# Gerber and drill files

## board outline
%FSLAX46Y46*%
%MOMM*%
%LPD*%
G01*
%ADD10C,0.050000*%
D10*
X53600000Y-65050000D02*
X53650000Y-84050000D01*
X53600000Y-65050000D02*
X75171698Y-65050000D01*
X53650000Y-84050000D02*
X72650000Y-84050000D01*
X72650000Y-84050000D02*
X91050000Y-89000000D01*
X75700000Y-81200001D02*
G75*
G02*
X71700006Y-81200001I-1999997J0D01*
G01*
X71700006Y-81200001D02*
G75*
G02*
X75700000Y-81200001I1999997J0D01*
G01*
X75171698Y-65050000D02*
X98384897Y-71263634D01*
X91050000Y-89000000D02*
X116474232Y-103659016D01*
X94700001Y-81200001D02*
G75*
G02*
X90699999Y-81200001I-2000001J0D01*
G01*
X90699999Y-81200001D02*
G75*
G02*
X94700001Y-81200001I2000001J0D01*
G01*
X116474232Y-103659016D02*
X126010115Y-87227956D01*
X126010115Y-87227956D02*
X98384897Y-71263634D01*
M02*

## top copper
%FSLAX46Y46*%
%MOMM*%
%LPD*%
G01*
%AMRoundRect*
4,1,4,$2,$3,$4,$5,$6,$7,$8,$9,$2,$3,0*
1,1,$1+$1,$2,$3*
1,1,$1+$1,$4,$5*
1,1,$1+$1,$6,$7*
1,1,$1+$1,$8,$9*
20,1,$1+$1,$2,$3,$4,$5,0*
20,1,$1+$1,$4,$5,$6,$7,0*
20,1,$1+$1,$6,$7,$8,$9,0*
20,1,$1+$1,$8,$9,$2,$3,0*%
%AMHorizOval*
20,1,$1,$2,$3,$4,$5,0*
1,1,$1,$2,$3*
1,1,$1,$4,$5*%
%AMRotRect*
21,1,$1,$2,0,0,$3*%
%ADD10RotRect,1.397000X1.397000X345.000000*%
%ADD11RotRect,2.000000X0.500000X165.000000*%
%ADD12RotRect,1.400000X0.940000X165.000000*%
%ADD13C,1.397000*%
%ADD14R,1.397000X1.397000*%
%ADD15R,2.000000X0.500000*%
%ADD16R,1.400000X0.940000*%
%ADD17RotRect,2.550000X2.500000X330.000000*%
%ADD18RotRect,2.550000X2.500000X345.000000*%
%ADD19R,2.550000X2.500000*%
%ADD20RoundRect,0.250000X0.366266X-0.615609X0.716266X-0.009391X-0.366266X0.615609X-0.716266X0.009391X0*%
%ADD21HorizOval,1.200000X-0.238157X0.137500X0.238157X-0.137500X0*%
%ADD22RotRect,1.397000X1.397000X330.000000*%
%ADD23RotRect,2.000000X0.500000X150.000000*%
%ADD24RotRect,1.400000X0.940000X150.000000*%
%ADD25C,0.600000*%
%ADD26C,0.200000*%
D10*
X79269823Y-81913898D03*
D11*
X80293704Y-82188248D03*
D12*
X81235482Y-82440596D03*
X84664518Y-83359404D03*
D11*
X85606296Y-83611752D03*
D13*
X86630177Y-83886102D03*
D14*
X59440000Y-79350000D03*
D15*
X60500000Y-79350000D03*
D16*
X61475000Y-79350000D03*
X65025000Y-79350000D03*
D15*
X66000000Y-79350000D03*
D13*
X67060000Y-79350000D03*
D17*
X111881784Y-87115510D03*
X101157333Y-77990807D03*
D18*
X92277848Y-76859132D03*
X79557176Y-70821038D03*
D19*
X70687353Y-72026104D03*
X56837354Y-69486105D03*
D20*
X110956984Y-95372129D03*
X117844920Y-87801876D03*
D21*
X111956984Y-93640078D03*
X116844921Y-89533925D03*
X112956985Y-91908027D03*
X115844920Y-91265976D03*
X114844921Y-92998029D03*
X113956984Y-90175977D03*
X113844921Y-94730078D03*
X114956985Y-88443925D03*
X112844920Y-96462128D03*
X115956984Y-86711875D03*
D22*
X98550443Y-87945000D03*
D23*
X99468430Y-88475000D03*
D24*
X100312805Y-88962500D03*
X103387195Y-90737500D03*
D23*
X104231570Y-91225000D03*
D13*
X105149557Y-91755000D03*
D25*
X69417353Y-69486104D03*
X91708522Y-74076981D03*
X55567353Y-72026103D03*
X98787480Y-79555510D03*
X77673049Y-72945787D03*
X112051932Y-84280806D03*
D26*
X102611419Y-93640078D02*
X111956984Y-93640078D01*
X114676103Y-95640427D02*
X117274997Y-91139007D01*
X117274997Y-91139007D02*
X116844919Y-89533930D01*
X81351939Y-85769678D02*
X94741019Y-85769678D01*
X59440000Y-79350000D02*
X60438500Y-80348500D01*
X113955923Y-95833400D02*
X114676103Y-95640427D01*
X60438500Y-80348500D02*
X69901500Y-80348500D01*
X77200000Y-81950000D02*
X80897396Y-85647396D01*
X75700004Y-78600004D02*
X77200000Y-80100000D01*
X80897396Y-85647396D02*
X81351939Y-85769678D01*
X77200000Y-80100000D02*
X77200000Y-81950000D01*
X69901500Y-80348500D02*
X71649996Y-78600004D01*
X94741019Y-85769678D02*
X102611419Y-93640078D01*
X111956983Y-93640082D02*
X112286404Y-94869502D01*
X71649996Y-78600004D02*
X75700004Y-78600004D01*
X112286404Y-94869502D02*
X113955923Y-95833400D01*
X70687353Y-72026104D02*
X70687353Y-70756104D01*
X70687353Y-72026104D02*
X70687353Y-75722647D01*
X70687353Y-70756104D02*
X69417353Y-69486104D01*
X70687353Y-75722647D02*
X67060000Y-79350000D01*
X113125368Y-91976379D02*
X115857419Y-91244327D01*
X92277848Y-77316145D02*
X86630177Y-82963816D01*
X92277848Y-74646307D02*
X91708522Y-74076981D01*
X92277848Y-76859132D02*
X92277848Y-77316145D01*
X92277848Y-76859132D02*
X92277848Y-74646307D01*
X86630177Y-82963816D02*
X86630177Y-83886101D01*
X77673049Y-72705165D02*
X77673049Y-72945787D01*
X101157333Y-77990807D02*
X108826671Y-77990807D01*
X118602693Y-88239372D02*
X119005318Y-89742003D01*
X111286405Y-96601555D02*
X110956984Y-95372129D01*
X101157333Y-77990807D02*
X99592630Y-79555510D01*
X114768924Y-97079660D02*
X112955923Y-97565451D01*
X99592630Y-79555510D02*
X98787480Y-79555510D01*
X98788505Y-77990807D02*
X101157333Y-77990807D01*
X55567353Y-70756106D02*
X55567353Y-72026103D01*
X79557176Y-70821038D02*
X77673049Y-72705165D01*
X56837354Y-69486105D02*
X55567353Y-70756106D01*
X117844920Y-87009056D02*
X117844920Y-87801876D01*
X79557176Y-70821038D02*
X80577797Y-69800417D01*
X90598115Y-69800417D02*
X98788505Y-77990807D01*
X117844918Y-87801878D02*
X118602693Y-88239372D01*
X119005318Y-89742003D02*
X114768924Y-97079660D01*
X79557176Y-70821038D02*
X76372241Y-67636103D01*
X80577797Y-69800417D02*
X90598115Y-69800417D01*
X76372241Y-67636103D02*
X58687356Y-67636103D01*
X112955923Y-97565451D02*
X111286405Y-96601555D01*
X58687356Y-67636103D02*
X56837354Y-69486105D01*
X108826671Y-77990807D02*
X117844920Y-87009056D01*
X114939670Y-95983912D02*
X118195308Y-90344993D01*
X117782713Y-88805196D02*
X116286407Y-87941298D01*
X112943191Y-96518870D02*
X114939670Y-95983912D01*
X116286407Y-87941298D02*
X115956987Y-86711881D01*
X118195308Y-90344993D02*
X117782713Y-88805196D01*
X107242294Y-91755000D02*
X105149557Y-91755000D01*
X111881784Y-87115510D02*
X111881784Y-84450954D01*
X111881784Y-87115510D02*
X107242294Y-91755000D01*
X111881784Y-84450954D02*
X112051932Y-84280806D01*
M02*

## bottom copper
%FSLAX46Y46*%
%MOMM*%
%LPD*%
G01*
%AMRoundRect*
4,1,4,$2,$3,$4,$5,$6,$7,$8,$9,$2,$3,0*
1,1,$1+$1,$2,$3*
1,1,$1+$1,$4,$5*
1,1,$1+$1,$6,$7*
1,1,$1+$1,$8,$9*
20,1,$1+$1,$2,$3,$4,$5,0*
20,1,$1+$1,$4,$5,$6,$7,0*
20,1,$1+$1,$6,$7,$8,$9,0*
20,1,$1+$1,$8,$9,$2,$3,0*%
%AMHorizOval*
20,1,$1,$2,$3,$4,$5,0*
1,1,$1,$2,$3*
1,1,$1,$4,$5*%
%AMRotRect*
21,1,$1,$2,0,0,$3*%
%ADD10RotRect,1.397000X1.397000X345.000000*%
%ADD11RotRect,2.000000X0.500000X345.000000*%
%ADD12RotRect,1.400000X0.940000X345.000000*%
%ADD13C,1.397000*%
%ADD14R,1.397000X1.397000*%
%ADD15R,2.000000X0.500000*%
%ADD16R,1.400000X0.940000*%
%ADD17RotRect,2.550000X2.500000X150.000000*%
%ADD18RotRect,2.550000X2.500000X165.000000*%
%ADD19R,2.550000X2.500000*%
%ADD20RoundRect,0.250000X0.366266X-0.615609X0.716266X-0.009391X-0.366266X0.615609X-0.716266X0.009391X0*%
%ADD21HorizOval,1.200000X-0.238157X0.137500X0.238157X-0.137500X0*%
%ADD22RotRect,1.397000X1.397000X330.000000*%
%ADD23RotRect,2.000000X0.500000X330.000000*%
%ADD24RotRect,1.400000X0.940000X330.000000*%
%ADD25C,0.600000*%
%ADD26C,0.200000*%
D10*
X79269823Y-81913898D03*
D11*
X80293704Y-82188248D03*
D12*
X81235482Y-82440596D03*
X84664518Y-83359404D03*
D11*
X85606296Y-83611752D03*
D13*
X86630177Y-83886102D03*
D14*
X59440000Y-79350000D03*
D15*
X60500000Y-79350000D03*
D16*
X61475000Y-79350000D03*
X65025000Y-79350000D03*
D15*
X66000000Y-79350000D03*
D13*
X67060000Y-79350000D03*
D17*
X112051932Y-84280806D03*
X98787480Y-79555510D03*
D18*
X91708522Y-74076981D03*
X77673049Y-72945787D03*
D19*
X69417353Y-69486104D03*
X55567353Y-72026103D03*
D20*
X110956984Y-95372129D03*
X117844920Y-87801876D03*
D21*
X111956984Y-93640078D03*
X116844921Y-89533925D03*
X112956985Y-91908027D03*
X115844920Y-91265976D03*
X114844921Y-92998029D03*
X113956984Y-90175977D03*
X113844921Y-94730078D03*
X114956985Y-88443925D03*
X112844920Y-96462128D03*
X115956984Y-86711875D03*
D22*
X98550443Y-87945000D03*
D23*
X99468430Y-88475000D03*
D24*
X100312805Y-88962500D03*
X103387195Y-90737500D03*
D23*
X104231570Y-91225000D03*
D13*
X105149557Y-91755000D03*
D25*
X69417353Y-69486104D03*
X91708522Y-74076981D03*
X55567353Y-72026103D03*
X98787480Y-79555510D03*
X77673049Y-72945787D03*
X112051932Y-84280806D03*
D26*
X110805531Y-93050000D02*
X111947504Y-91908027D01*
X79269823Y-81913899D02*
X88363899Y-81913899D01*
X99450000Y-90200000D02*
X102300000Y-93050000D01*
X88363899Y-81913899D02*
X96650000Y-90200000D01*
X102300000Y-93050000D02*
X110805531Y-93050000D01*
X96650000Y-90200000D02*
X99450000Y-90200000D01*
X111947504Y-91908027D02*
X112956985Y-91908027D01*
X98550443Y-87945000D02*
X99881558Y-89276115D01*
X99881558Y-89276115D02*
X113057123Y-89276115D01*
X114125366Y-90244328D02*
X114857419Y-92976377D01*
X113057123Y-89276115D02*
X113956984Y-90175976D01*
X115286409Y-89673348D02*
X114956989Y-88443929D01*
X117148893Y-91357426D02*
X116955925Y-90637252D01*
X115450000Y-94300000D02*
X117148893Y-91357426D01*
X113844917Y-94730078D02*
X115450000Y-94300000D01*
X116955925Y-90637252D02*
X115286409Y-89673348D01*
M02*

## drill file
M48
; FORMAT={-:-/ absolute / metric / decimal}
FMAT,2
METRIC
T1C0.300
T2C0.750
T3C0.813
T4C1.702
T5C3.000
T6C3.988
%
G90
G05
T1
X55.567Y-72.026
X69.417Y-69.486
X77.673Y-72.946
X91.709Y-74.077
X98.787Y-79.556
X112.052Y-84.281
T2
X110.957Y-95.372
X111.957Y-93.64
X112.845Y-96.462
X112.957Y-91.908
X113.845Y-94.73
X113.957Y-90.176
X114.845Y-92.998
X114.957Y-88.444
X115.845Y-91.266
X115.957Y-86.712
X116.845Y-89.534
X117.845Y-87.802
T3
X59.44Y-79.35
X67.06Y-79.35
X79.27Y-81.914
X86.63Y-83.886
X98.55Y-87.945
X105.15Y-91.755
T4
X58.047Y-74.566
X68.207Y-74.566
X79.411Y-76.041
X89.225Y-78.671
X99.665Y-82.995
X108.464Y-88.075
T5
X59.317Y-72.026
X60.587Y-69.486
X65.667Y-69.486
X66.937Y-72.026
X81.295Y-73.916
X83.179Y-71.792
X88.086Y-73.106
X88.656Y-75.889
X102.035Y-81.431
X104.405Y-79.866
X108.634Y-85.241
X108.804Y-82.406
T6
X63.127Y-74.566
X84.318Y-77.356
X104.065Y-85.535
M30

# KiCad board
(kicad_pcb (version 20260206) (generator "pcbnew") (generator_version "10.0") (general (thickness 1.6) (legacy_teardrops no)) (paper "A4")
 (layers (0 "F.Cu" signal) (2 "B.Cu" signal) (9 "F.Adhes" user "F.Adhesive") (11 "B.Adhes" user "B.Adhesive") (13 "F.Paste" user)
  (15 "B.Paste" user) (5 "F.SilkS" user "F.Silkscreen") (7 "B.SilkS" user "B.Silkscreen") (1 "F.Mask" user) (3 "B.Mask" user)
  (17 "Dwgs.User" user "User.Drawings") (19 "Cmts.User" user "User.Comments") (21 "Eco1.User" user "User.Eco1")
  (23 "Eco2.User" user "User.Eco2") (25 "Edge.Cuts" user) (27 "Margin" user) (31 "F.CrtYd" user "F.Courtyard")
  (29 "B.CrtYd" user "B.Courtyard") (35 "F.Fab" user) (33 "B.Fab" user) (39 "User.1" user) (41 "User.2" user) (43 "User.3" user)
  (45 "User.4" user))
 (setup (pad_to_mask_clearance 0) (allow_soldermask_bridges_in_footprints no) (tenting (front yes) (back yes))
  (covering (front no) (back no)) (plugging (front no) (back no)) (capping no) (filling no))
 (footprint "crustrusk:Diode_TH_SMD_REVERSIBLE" (layer "F.Cu") (at 82.95 82.9 -15)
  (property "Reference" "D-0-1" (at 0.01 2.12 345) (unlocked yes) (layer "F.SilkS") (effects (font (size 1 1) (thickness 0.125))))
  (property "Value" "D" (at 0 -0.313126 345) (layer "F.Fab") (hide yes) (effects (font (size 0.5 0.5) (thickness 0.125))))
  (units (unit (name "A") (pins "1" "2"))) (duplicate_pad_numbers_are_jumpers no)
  (pad "1" thru_hole rect (at -3.81 -0.000001 345) (size 1.397 1.397) (drill 0.8128) (layers "*.Cu" "*.Mask") (remove_unused_layers no)
   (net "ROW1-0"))
  (pad "1" smd rect (at -2.75 0 165) (size 2 0.5) (layers "F.Cu") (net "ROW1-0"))
  (pad "1" smd rect (at -2.75 0 345) (size 2 0.5) (layers "B.Cu") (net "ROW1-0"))
  (pad "1" smd rect (at -1.775 0 165) (size 1.4 0.94) (layers "F.Cu" "F.Mask" "F.Paste") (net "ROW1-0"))
  (pad "1" smd rect (at -1.775 0 345) (size 1.4 0.94) (layers "B.Cu" "B.Mask" "B.Paste") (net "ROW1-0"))
  (pad "2" smd rect (at 1.775 0 165) (size 1.4 0.94) (layers "F.Cu" "F.Mask" "F.Paste") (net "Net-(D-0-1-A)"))
  (pad "2" smd rect (at 1.775 0 345) (size 1.4 0.94) (layers "B.Cu" "B.Mask" "B.Paste") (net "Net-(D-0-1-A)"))
  (pad "2" smd rect (at 2.75 0 165) (size 2 0.5) (layers "F.Cu") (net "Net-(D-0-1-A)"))
  (pad "2" smd rect (at 2.75 0 345) (size 2 0.5) (layers "B.Cu") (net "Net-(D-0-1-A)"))
  (pad "2" thru_hole circle (at 3.81 0.000001 345) (size 1.397 1.397) (drill 0.8128) (layers "*.Cu" "*.Mask") (remove_unused_layers no)
   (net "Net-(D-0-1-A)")))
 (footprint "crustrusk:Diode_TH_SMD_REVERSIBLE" (layer "F.Cu") (at 63.25 79.35)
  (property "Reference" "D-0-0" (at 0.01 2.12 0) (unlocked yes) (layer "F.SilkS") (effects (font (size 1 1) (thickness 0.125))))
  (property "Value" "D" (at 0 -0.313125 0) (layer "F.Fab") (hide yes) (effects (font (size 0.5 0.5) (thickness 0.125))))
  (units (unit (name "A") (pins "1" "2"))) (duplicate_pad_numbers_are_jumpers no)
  (pad "1" thru_hole rect (at -3.81 0) (size 1.397 1.397) (drill 0.8128) (layers "*.Cu" "*.Mask") (remove_unused_layers no) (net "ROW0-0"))
  (pad "1" smd rect (at -2.75 0 180) (size 2 0.5) (layers "F.Cu") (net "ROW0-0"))
  (pad "1" smd rect (at -2.75 0) (size 2 0.5) (layers "B.Cu") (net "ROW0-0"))
  (pad "1" smd rect (at -1.775 0 180) (size 1.4 0.94) (layers "F.Cu" "F.Mask" "F.Paste") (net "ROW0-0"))
  (pad "1" smd rect (at -1.775 0) (size 1.4 0.94) (layers "B.Cu" "B.Mask" "B.Paste") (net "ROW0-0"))
  (pad "2" smd rect (at 1.775 0 180) (size 1.4 0.94) (layers "F.Cu" "F.Mask" "F.Paste") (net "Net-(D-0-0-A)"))
  (pad "2" smd rect (at 1.775 0) (size 1.4 0.94) (layers "B.Cu" "B.Mask" "B.Paste") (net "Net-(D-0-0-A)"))
  (pad "2" smd rect (at 2.75 0 180) (size 2 0.5) (layers "F.Cu") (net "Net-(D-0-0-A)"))
  (pad "2" smd rect (at 2.75 0) (size 2 0.5) (layers "B.Cu") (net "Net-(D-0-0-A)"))
  (pad "2" thru_hole circle (at 3.81 0) (size 1.397 1.397) (drill 0.8128) (layers "*.Cu" "*.Mask") (remove_unused_layers no)
   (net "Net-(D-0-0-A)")))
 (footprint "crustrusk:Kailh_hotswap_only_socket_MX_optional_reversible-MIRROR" (layer "F.Cu") (at 104.064632 85.535215 -30)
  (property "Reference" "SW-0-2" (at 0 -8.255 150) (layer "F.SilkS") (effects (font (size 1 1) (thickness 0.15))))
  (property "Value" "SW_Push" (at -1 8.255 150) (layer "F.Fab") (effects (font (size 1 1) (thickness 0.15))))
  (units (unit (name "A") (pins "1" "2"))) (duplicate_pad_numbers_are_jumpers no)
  (pad "" np_thru_hole circle (at -5.08 0 330) (size 1.7018 1.7018) (drill 1.7018) (layers "*.Cu" "*.Mask"))
  (pad "" np_thru_hole circle (at -3.81 -2.54 150) (size 3 3) (drill 3) (layers "*.Cu" "*.Mask"))
  (pad "" np_thru_hole circle (at -2.54 -5.079997 330) (size 3 3) (drill 3) (layers "*.Cu" "*.Mask"))
  (pad "" np_thru_hole circle (at 0 0 330) (size 3.9878 3.9878) (drill 3.9878) (layers "*.Cu" "*.Mask"))
  (pad "" np_thru_hole circle (at 2.540002 -5.080001 150) (size 3 3) (drill 3) (layers "*.Cu" "*.Mask"))
  (pad "" np_thru_hole circle (at 3.81 -2.540001 330) (size 3 3) (drill 3) (layers "*.Cu" "*.Mask"))
  (pad "" np_thru_hole circle (at 5.08 0 330) (size 1.7018 1.7018) (drill 1.7018) (layers "*.Cu" "*.Mask"))
  (pad "1" smd rect (at 6.29 -5.08 150) (size 2.55 2.5) (layers "B.Cu" "B.Mask" "B.Paste") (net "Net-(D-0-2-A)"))
  (pad "1" smd rect (at 7.56 -2.54 330) (size 2.55 2.5) (layers "F.Cu" "F.Mask" "F.Paste") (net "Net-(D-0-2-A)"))
  (pad "2" smd rect (at -7.56 -2.54 150) (size 2.55 2.5) (layers "B.Cu" "B.Mask" "B.Paste") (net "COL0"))
  (pad "2" smd rect (at -6.289999 -5.079999 330) (size 2.55 2.5) (layers "F.Cu" "F.Mask" "F.Paste") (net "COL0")))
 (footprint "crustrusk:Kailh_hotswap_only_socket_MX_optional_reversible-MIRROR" (layer "F.Cu") (at 84.318048 77.355912 -15)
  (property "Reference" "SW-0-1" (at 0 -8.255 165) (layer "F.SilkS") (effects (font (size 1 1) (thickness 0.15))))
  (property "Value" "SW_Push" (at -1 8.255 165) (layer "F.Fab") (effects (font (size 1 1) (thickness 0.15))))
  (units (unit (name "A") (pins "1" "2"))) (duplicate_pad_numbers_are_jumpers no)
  (pad "" np_thru_hole circle (at -5.08 0 345) (size 1.7018 1.7018) (drill 1.7018) (layers "*.Cu" "*.Mask"))
  (pad "" np_thru_hole circle (at -3.81 -2.54 165) (size 3 3) (drill 3) (layers "*.Cu" "*.Mask"))
  (pad "" np_thru_hole circle (at -2.54 -5.079998 345) (size 3 3) (drill 3) (layers "*.Cu" "*.Mask"))
  (pad "" np_thru_hole circle (at 0 0 345) (size 3.9878 3.9878) (drill 3.9878) (layers "*.Cu" "*.Mask"))
  (pad "" np_thru_hole circle (at 2.540003 -5.080001 165) (size 3 3) (drill 3) (layers "*.Cu" "*.Mask"))
  (pad "" np_thru_hole circle (at 3.81 -2.54 345) (size 3 3) (drill 3) (layers "*.Cu" "*.Mask"))
  (pad "" np_thru_hole circle (at 5.08 0 345) (size 1.7018 1.7018) (drill 1.7018) (layers "*.Cu" "*.Mask"))
  (pad "1" smd rect (at 6.29 -5.08 165) (size 2.55 2.5) (layers "B.Cu" "B.Mask" "B.Paste") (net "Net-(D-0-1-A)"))
  (pad "1" smd rect (at 7.56 -2.54 345) (size 2.55 2.5) (layers "F.Cu" "F.Mask" "F.Paste") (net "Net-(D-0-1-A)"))
  (pad "2" smd rect (at -7.56 -2.540001 165) (size 2.55 2.5) (layers "B.Cu" "B.Mask" "B.Paste") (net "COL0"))
  (pad "2" smd rect (at -6.289999 -5.079999 345) (size 2.55 2.5) (layers "F.Cu" "F.Mask" "F.Paste") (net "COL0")))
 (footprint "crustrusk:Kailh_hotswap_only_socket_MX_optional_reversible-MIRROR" (layer "F.Cu") (at 63.127353 74.566104)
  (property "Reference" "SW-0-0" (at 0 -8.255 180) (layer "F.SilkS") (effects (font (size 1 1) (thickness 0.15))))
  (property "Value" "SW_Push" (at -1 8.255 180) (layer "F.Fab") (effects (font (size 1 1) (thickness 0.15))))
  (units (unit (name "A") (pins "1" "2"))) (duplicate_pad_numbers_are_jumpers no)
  (pad "" np_thru_hole circle (at -5.08 0) (size 1.7018 1.7018) (drill 1.7018) (layers "*.Cu" "*.Mask"))
  (pad "" np_thru_hole circle (at -3.81 -2.54 180) (size 3 3) (drill 3) (layers "*.Cu" "*.Mask"))
  (pad "" np_thru_hole circle (at -2.54 -5.079998) (size 3 3) (drill 3) (layers "*.Cu" "*.Mask"))
  (pad "" np_thru_hole circle (at 0 0) (size 3.9878 3.9878) (drill 3.9878) (layers "*.Cu" "*.Mask"))
  (pad "" np_thru_hole circle (at 2.540002 -5.080001 180) (size 3 3) (drill 3) (layers "*.Cu" "*.Mask"))
  (pad "" np_thru_hole circle (at 3.81 -2.54) (size 3 3) (drill 3) (layers "*.Cu" "*.Mask"))
  (pad "" np_thru_hole circle (at 5.08 0) (size 1.7018 1.7018) (drill 1.7018) (layers "*.Cu" "*.Mask"))
  (pad "1" smd rect (at 6.29 -5.08 180) (size 2.55 2.5) (layers "B.Cu" "B.Mask" "B.Paste") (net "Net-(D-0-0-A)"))
  (pad "1" smd rect (at 7.56 -2.54) (size 2.55 2.5) (layers "F.Cu" "F.Mask" "F.Paste") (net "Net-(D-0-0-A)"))
  (pad "2" smd rect (at -7.56 -2.540001 180) (size 2.55 2.5) (layers "B.Cu" "B.Mask" "B.Paste") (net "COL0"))
  (pad "2" smd rect (at -6.289999 -5.079999) (size 2.55 2.5) (layers "F.Cu" "F.Mask" "F.Paste") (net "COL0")))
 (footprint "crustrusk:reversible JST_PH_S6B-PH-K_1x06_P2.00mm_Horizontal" (layer "F.Cu") (at 110.956984 95.372129 60)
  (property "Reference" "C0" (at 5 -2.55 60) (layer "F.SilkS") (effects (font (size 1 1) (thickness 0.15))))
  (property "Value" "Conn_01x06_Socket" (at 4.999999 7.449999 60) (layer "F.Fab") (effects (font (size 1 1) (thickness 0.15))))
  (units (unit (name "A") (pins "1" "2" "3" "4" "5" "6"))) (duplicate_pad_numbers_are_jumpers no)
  (pad "1" thru_hole roundrect (at 0 0 60) (size 1.2 1.75) (drill 0.75) (layers "*.Cu" "*.Mask") (remove_unused_layers no)
   (roundrect_rratio 0.208333) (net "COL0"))
  (pad "1" thru_hole roundrect (at 9.999999 2.180001 60) (size 1.2 1.75) (drill 0.75) (layers "*.Cu" "*.Mask") (remove_unused_layers no)
   (roundrect_rratio 0.208333) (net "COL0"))
  (pad "2" thru_hole oval (at 2 0 60) (size 1.2 1.75) (drill 0.75) (layers "*.Cu" "*.Mask") (remove_unused_layers no) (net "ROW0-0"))
  (pad "2" thru_hole oval (at 8.000001 2.180001 60) (size 1.2 1.75) (drill 0.75) (layers "*.Cu" "*.Mask") (remove_unused_layers no)
   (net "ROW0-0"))
  (pad "3" thru_hole oval (at 4.000001 0.000001 60) (size 1.2 1.75) (drill 0.75) (layers "*.Cu" "*.Mask") (remove_unused_layers no)
   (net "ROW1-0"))
  (pad "3" thru_hole oval (at 6.000001 2.18 60) (size 1.2 1.75) (drill 0.75) (layers "*.Cu" "*.Mask") (remove_unused_layers no)
   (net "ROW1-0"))
  (pad "4" thru_hole oval (at 3.999999 2.180002 60) (size 1.2 1.75) (drill 0.75) (layers "*.Cu" "*.Mask") (remove_unused_layers no)
   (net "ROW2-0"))
  (pad "4" thru_hole oval (at 6 0 60) (size 1.2 1.75) (drill 0.75) (layers "*.Cu" "*.Mask") (remove_unused_layers no) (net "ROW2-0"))
  (pad "5" thru_hole oval (at 2.000001 2.180001 60) (size 1.2 1.75) (drill 0.75) (layers "*.Cu" "*.Mask") (remove_unused_layers no)
   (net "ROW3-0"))
  (pad "5" thru_hole oval (at 8.000001 0 60) (size 1.2 1.75) (drill 0.75) (layers "*.Cu" "*.Mask") (remove_unused_layers no) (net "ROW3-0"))
  (pad "6" thru_hole oval (at 0.000001 2.18 60) (size 1.2 1.75) (drill 0.75) (layers "*.Cu" "*.Mask") (remove_unused_layers no)
   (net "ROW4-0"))
  (pad "6" thru_hole oval (at 10 0 60) (size 1.2 1.75) (drill 0.75) (layers "*.Cu" "*.Mask") (remove_unused_layers no) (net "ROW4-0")))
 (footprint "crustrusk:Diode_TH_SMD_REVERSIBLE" (layer "F.Cu") (at 101.85 89.85 -30)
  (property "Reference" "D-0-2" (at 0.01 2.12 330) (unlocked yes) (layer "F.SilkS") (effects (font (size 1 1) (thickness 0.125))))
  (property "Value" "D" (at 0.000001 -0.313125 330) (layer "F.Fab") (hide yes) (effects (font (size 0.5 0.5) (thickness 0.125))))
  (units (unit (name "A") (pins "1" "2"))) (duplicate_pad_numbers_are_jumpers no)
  (pad "1" thru_hole rect (at -3.81 0 330) (size 1.397 1.397) (drill 0.8128) (layers "*.Cu" "*.Mask") (remove_unused_layers no)
   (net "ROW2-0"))
  (pad "1" smd rect (at -2.75 0 150) (size 2 0.5) (layers "F.Cu") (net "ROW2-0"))
  (pad "1" smd rect (at -2.75 0 330) (size 2 0.5) (layers "B.Cu") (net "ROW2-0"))
  (pad "1" smd rect (at -1.775 0 150) (size 1.4 0.94) (layers "F.Cu" "F.Mask" "F.Paste") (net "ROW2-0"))
  (pad "1" smd rect (at -1.775 0 330) (size 1.4 0.94) (layers "B.Cu" "B.Mask" "B.Paste") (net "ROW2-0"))
  (pad "2" smd rect (at 1.775 0 150) (size 1.4 0.94) (layers "F.Cu" "F.Mask" "F.Paste") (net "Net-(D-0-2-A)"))
  (pad "2" smd rect (at 1.775 0 330) (size 1.4 0.94) (layers "B.Cu" "B.Mask" "B.Paste") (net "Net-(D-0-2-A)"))
  (pad "2" smd rect (at 2.75 0 150) (size 2 0.5) (layers "F.Cu") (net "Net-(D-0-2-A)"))
  (pad "2" smd rect (at 2.75 0 330) (size 2 0.5) (layers "B.Cu") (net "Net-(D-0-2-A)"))
  (pad "2" thru_hole circle (at 3.81 0 330) (size 1.397 1.397) (drill 0.8128) (layers "*.Cu" "*.Mask") (remove_unused_layers no)
   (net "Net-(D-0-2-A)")))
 (gr_line (start 53.6 65.05) (end 53.65 84.05) (stroke (width 0.05) (type default)) (layer "Edge.Cuts"))
 (gr_line (start 53.6 65.05) (end 75.171698 65.05) (stroke (width 0.05) (type default)) (layer "Edge.Cuts"))
 (gr_line (start 53.65 84.05) (end 72.65 84.05) (stroke (width 0.05) (type default)) (layer "Edge.Cuts"))
 (gr_line (start 72.65 84.05) (end 91.05 89) (stroke (width 0.05) (type default)) (layer "Edge.Cuts"))
 (gr_circle (center 73.700003 81.200001) (end 75.7 81.200001) (stroke (width 0.05) (type default)) (fill no) (layer "Edge.Cuts"))
 (gr_line (start 75.171698 65.05) (end 98.384897 71.263634) (stroke (width 0.05) (type default)) (layer "Edge.Cuts"))
 (gr_line (start 91.05 89) (end 116.474232 103.659016) (stroke (width 0.05) (type default)) (layer "Edge.Cuts"))
 (gr_circle (center 92.7 81.200001) (end 94.700001 81.200001) (stroke (width 0.05) (type default)) (fill no) (layer "Edge.Cuts"))
 (gr_line (start 116.474232 103.659016) (end 126.010115 87.227956) (stroke (width 0.05) (type default)) (layer "Edge.Cuts"))
 (gr_line (start 126.010115 87.227956) (end 98.384897 71.263634) (stroke (width 0.05) (type default)) (layer "Edge.Cuts"))
 (segment (start 102.611419 93.640078) (end 111.956984 93.640078) (width 0.2) (layer "F.Cu") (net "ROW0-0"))
 (segment (start 114.676103 95.640427) (end 117.274997 91.139007) (width 0.2) (layer "F.Cu") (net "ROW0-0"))
 (segment (start 117.274997 91.139007) (end 116.844919 89.53393) (width 0.2) (layer "F.Cu") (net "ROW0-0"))
 (segment (start 81.351939 85.769678) (end 94.741019 85.769678) (width 0.2) (layer "F.Cu") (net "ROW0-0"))
 (segment (start 59.44 79.35) (end 60.4385 80.3485) (width 0.2) (layer "F.Cu") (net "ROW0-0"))
 (segment (start 113.955923 95.8334) (end 114.676103 95.640427) (width 0.2) (layer "F.Cu") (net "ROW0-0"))
 (segment (start 60.4385 80.3485) (end 69.9015 80.3485) (width 0.2) (layer "F.Cu") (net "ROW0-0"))
 (segment (start 77.2 81.95) (end 80.897396 85.647396) (width 0.2) (layer "F.Cu") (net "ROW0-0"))
 (segment (start 75.700004 78.600004) (end 77.2 80.1) (width 0.2) (layer "F.Cu") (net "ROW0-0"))
 (segment (start 80.897396 85.647396) (end 81.351939 85.769678) (width 0.2) (layer "F.Cu") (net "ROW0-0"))
 (segment (start 77.2 80.1) (end 77.2 81.95) (width 0.2) (layer "F.Cu") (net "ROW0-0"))
 (segment (start 69.9015 80.3485) (end 71.649996 78.600004) (width 0.2) (layer "F.Cu") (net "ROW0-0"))
 (segment (start 94.741019 85.769678) (end 102.611419 93.640078) (width 0.2) (layer "F.Cu") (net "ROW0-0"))
 (segment (start 111.956983 93.640082) (end 112.286404 94.869502) (width 0.2) (layer "F.Cu") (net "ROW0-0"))
 (segment (start 71.649996 78.600004) (end 75.700004 78.600004) (width 0.2) (layer "F.Cu") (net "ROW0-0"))
 (segment (start 112.286404 94.869502) (end 113.955923 95.8334) (width 0.2) (layer "F.Cu") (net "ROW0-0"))
 (segment (start 70.687353 72.026104) (end 70.687353 70.756104) (width 0.2) (layer "F.Cu") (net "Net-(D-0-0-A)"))
 (segment (start 70.687353 72.026104) (end 70.687353 75.722647) (width 0.2) (layer "F.Cu") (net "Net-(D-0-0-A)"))
 (segment (start 70.687353 70.756104) (end 69.417353 69.486104) (width 0.2) (layer "F.Cu") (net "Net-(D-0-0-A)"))
 (segment (start 70.687353 75.722647) (end 67.06 79.35) (width 0.2) (layer "F.Cu") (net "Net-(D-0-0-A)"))
 (via (at 69.417353 69.486104) (size 0.6) (drill 0.3) (layers "F.Cu" "B.Cu") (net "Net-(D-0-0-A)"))
 (segment (start 113.125368 91.976379) (end 115.857419 91.244327) (width 0.2) (layer "F.Cu") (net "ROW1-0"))
 (segment (start 110.805531 93.05) (end 111.947504 91.908027) (width 0.2) (layer "B.Cu") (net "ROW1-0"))
 (segment (start 79.269823 81.913899) (end 88.363899 81.913899) (width 0.2) (layer "B.Cu") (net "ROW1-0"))
 (segment (start 99.45 90.2) (end 102.3 93.05) (width 0.2) (layer "B.Cu") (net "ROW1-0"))
 (segment (start 88.363899 81.913899) (end 96.65 90.2) (width 0.2) (layer "B.Cu") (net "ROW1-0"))
 (segment (start 102.3 93.05) (end 110.805531 93.05) (width 0.2) (layer "B.Cu") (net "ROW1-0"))
 (segment (start 96.65 90.2) (end 99.45 90.2) (width 0.2) (layer "B.Cu") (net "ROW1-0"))
 (segment (start 111.947504 91.908027) (end 112.956985 91.908027) (width 0.2) (layer "B.Cu") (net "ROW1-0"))
 (segment (start 92.277848 77.316145) (end 86.630177 82.963816) (width 0.2) (layer "F.Cu") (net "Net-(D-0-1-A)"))
 (segment (start 92.277848 74.646307) (end 91.708522 74.076981) (width 0.2) (layer "F.Cu") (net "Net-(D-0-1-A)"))
 (segment (start 92.277848 76.859132) (end 92.277848 77.316145) (width 0.2) (layer "F.Cu") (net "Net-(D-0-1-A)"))
 (segment (start 92.277848 76.859132) (end 92.277848 74.646307) (width 0.2) (layer "F.Cu") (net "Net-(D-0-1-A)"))
 (segment (start 86.630177 82.963816) (end 86.630177 83.886101) (width 0.2) (layer "F.Cu") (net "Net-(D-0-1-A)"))
 (via (at 91.708522 74.076981) (size 0.6) (drill 0.3) (layers "F.Cu" "B.Cu") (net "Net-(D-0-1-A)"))
 (segment (start 77.673049 72.705165) (end 77.673049 72.945787) (width 0.2) (layer "F.Cu") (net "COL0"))
 (segment (start 101.157333 77.990807) (end 108.826671 77.990807) (width 0.2) (layer "F.Cu") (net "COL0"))
 (segment (start 118.602693 88.239372) (end 119.005318 89.742003) (width 0.2) (layer "F.Cu") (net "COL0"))
 (segment (start 111.286405 96.601555) (end 110.956984 95.372129) (width 0.2) (layer "F.Cu") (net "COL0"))
 (segment (start 101.157333 77.990807) (end 99.59263 79.55551) (width 0.2) (layer "F.Cu") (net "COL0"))
 (segment (start 114.768924 97.07966) (end 112.955923 97.565451) (width 0.2) (layer "F.Cu") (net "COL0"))
 (segment (start 99.59263 79.55551) (end 98.78748 79.55551) (width 0.2) (layer "F.Cu") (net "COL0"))
 (segment (start 98.788505 77.990807) (end 101.157333 77.990807) (width 0.2) (layer "F.Cu") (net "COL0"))
 (segment (start 55.567353 70.756106) (end 55.567353 72.026103) (width 0.2) (layer "F.Cu") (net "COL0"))
 (segment (start 79.557176 70.821038) (end 77.673049 72.705165) (width 0.2) (layer "F.Cu") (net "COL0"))
 (segment (start 56.837354 69.486105) (end 55.567353 70.756106) (width 0.2) (layer "F.Cu") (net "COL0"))
 (segment (start 117.84492 87.009056) (end 117.84492 87.801876) (width 0.2) (layer "F.Cu") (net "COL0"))
 (segment (start 79.557176 70.821038) (end 80.577797 69.800417) (width 0.2) (layer "F.Cu") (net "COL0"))
 (segment (start 90.598115 69.800417) (end 98.788505 77.990807) (width 0.2) (layer "F.Cu") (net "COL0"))
 (segment (start 117.844918 87.801878) (end 118.602693 88.239372) (width 0.2) (layer "F.Cu") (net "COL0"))
 (segment (start 119.005318 89.742003) (end 114.768924 97.07966) (width 0.2) (layer "F.Cu") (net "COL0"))
 (segment (start 79.557176 70.821038) (end 76.372241 67.636103) (width 0.2) (layer "F.Cu") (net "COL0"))
 (segment (start 80.577797 69.800417) (end 90.598115 69.800417) (width 0.2) (layer "F.Cu") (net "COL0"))
 (segment (start 76.372241 67.636103) (end 58.687356 67.636103) (width 0.2) (layer "F.Cu") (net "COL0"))
 (segment (start 112.955923 97.565451) (end 111.286405 96.601555) (width 0.2) (layer "F.Cu") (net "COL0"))
 (segment (start 58.687356 67.636103) (end 56.837354 69.486105) (width 0.2) (layer "F.Cu") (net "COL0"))
 (segment (start 108.826671 77.990807) (end 117.84492 87.009056) (width 0.2) (layer "F.Cu") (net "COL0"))
 (via (at 55.567353 72.026103) (size 0.6) (drill 0.3) (layers "F.Cu" "B.Cu") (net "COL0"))
 (via (at 98.78748 79.55551) (size 0.6) (drill 0.3) (layers "F.Cu" "B.Cu") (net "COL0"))
 (via (at 77.673049 72.945787) (size 0.6) (drill 0.3) (layers "F.Cu" "B.Cu") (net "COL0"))
 (segment (start 98.550443 87.945) (end 99.881558 89.276115) (width 0.2) (layer "B.Cu") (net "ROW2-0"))
 (segment (start 99.881558 89.276115) (end 113.057123 89.276115) (width 0.2) (layer "B.Cu") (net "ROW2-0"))
 (segment (start 114.125366 90.244328) (end 114.857419 92.976377) (width 0.2) (layer "B.Cu") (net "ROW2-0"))
 (segment (start 113.057123 89.276115) (end 113.956984 90.175976) (width 0.2) (layer "B.Cu") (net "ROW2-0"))
 (segment (start 115.286409 89.673348) (end 114.956989 88.443929) (width 0.2) (layer "B.Cu") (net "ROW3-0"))
 (segment (start 117.148893 91.357426) (end 116.955925 90.637252) (width 0.2) (layer "B.Cu") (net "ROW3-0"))
 (segment (start 115.45 94.3) (end 117.148893 91.357426) (width 0.2) (layer "B.Cu") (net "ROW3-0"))
 (segment (start 113.844917 94.730078) (end 115.45 94.3) (width 0.2) (layer "B.Cu") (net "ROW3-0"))
 (segment (start 116.955925 90.637252) (end 115.286409 89.673348) (width 0.2) (layer "B.Cu") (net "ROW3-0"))
 (segment (start 114.93967 95.983912) (end 118.195308 90.344993) (width 0.2) (layer "F.Cu") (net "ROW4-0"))
 (segment (start 117.782713 88.805196) (end 116.286407 87.941298) (width 0.2) (layer "F.Cu") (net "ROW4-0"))
 (segment (start 112.943191 96.51887) (end 114.93967 95.983912) (width 0.2) (layer "F.Cu") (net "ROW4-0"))
 (segment (start 116.286407 87.941298) (end 115.956987 86.711881) (width 0.2) (layer "F.Cu") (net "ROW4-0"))
 (segment (start 118.195308 90.344993) (end 117.782713 88.805196) (width 0.2) (layer "F.Cu") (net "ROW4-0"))
 (segment (start 107.242294 91.755) (end 105.149557 91.755) (width 0.2) (layer "F.Cu") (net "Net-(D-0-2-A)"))
 (segment (start 111.881784 87.11551) (end 111.881784 84.450954) (width 0.2) (layer "F.Cu") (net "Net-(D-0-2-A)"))
 (segment (start 111.881784 87.11551) (end 107.242294 91.755) (width 0.2) (layer "F.Cu") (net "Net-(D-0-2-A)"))
 (segment (start 111.881784 84.450954) (end 112.051932 84.280806) (width 0.2) (layer "F.Cu") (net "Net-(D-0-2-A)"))
 (via (at 112.051932 84.280806) (size 0.6) (drill 0.3) (layers "F.Cu" "B.Cu") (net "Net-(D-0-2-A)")))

